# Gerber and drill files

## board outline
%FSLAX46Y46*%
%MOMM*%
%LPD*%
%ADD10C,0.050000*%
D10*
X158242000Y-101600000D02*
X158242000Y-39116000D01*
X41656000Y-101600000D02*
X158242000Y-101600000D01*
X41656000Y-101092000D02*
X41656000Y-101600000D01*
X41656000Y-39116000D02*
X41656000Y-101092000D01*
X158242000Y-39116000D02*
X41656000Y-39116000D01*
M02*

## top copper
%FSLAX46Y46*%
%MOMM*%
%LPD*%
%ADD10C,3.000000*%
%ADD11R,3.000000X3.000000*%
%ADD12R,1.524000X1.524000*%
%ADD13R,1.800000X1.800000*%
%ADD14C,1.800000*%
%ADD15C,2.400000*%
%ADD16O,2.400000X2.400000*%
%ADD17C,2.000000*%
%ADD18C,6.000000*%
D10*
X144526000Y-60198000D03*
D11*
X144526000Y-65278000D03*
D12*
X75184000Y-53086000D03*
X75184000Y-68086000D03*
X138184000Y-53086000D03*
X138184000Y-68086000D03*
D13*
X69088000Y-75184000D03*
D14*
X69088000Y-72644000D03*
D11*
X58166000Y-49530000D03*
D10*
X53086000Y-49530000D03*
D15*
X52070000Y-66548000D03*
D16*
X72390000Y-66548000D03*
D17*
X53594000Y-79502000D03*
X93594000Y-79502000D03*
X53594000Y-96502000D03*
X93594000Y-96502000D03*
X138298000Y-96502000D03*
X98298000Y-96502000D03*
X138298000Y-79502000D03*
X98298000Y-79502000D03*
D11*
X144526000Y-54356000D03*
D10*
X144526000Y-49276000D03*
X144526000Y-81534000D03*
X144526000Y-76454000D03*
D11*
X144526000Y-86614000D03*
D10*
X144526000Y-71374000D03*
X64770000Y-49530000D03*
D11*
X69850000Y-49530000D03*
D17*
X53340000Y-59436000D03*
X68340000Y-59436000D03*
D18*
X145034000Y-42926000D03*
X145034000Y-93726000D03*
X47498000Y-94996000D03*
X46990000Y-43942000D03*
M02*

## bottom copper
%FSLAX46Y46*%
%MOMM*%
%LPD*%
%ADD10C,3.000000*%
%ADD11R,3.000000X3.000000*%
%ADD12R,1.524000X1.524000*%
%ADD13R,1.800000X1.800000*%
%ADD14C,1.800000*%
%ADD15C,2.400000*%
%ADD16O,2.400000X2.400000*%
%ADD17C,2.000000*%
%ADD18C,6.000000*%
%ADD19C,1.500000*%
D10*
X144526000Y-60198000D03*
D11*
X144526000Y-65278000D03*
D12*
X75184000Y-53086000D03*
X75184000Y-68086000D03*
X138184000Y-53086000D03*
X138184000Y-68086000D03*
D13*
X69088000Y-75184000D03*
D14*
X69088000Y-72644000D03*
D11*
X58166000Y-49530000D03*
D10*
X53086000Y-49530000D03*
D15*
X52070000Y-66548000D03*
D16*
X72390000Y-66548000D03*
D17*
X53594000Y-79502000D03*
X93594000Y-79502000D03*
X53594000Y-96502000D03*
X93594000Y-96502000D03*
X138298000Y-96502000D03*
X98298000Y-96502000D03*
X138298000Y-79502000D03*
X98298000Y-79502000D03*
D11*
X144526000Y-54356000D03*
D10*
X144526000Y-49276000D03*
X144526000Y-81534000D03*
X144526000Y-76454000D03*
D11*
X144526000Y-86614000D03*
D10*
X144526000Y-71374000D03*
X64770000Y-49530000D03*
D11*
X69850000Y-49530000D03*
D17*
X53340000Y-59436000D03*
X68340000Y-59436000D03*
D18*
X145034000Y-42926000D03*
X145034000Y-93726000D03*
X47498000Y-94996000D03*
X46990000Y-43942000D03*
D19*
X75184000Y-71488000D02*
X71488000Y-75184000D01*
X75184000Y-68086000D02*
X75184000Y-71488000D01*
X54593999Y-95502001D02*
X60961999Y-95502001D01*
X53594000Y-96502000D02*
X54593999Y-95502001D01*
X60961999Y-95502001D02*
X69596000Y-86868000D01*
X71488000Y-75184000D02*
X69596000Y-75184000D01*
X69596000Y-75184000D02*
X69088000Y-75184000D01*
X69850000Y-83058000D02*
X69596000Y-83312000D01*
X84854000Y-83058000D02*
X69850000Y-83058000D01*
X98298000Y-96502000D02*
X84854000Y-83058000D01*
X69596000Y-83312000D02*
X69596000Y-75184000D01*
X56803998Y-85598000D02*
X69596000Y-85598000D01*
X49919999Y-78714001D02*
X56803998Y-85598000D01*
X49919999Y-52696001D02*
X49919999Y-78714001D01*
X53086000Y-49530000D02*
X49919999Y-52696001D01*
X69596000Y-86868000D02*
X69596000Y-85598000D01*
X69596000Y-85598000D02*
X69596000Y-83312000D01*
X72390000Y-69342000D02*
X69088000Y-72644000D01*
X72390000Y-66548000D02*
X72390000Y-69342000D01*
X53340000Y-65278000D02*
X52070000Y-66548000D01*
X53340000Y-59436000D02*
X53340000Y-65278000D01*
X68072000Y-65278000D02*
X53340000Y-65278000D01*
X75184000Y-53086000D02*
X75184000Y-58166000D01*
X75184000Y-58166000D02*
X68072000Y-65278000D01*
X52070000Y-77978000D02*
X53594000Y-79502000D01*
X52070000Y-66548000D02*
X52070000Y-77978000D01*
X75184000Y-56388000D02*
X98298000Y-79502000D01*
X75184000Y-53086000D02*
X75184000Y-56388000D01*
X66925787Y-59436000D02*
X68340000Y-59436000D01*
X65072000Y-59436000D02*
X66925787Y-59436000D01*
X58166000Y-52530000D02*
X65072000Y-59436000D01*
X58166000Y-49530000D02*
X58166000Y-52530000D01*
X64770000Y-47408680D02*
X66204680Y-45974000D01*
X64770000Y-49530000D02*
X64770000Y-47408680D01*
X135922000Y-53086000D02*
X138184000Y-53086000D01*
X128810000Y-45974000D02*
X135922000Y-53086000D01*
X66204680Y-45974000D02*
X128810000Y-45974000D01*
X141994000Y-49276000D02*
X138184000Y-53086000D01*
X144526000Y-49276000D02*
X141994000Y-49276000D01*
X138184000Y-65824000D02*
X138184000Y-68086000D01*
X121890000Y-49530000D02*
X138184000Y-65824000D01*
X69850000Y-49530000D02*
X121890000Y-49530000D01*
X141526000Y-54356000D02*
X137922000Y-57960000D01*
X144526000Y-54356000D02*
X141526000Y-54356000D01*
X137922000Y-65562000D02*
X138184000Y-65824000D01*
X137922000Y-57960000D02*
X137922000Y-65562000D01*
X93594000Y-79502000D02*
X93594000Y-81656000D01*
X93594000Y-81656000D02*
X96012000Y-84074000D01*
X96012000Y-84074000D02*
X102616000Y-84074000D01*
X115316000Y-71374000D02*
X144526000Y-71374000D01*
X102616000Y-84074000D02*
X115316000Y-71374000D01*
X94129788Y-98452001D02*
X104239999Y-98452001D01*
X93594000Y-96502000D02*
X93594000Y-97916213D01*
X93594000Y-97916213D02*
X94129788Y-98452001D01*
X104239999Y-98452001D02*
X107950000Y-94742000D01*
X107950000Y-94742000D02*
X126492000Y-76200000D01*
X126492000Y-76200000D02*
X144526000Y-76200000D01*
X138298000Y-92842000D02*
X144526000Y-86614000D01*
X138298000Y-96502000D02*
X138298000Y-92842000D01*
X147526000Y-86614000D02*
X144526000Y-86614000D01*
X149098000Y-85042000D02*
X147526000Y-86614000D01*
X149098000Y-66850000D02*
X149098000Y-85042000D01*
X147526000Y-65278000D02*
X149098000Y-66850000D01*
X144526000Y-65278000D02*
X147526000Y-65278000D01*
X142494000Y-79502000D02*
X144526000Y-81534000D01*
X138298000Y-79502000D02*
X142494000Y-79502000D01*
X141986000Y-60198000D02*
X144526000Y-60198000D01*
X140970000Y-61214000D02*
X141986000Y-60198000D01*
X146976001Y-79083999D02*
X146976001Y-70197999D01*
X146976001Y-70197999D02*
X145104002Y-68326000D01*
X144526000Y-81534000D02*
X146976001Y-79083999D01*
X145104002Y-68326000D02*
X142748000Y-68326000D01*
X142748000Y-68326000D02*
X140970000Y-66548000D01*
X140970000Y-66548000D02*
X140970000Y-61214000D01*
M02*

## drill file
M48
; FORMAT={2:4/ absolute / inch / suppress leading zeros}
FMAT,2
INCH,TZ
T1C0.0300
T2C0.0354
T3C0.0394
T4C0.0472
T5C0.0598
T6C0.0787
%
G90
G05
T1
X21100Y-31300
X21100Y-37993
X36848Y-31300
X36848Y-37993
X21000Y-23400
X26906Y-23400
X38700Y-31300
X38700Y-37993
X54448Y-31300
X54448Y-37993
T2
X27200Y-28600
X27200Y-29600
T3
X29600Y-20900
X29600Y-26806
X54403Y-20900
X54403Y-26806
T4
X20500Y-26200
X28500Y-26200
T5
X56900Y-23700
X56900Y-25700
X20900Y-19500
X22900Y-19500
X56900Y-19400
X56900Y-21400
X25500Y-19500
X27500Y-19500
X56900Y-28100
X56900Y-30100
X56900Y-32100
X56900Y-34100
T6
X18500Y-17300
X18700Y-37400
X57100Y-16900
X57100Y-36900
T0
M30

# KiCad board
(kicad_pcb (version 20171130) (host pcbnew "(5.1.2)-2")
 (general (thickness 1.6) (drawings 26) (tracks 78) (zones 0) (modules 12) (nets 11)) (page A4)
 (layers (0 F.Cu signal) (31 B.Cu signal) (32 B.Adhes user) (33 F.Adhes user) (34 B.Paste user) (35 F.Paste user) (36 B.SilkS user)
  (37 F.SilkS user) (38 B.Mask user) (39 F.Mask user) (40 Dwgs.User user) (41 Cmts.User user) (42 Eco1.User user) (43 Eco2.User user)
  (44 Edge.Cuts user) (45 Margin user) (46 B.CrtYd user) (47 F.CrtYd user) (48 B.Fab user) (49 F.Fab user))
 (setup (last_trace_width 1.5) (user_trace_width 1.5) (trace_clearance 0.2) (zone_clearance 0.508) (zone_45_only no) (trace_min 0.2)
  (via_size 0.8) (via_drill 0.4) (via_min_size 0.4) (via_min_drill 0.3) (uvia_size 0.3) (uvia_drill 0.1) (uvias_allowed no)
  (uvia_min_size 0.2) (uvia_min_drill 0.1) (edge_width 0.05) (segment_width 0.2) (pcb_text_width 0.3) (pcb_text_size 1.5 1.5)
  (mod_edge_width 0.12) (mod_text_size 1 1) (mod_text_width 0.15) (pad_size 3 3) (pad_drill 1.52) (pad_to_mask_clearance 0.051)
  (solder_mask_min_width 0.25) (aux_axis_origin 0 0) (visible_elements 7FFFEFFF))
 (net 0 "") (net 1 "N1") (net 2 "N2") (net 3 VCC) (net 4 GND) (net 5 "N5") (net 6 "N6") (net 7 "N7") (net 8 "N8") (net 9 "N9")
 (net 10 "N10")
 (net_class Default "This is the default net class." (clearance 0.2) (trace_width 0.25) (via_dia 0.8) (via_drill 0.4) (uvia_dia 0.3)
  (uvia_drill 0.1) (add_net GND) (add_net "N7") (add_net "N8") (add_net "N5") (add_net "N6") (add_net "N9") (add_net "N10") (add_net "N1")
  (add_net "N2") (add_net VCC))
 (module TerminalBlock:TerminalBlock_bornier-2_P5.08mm (layer F.Cu) (at 144.526 65.278 90)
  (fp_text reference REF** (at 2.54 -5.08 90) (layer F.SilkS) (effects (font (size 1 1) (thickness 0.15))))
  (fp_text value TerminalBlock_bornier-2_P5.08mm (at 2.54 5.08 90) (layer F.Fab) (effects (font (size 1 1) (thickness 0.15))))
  (pad 2 thru_hole circle (at 5.08 0 90) (size 3 3) (drill 1.52) (layers *.Cu *.Mask) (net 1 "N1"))
  (pad 1 thru_hole rect (at 0 0 90) (size 3 3) (drill 1.52) (layers *.Cu *.Mask) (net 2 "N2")))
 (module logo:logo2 (layer F.Cu) (at 105.918 60.198)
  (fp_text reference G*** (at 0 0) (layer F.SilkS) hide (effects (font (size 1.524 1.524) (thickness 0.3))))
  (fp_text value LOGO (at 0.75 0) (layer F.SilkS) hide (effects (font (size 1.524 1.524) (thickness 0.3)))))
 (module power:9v (layer F.Cu) (at 75.184 53.086)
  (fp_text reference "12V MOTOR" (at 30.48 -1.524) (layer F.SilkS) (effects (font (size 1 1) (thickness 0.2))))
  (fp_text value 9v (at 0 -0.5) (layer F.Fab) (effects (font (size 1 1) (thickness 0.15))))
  (pad 1 thru_hole rect (at 0 0) (size 1.524 1.524) (drill 1) (layers *.Cu *.Mask) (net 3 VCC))
  (pad 3 thru_hole rect (at 0 15) (size 1.524 1.524) (drill 1) (layers *.Cu *.Mask) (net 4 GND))
  (pad 2 thru_hole rect (at 63 0) (size 1.524 1.524) (drill 1) (layers *.Cu *.Mask) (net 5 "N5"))
  (pad 4 thru_hole rect (at 63 15) (size 1.524 1.524) (drill 1) (layers *.Cu *.Mask) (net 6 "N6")))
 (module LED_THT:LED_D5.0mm (layer F.Cu) (at 69.088 75.184 90)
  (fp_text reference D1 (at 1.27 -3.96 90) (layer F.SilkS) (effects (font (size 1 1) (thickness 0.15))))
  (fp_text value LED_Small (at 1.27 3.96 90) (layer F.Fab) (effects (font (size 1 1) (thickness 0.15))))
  (pad 1 thru_hole rect (at 0 0 90) (size 1.8 1.8) (drill 0.9) (layers *.Cu *.Mask) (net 4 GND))
  (pad 2 thru_hole circle (at 2.54 0 90) (size 1.8 1.8) (drill 0.9) (layers *.Cu *.Mask) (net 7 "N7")))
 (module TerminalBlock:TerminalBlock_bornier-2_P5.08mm (layer F.Cu) (at 58.166 49.53 180)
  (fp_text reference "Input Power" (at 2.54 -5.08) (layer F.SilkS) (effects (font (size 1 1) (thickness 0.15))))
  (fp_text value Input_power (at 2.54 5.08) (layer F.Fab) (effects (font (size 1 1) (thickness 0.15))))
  (pad 1 thru_hole rect (at 0 0 180) (size 3 3) (drill 1.52) (layers *.Cu *.Mask) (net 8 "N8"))
  (pad 2 thru_hole circle (at 5.08 0 180) (size 3 3) (drill 1.52) (layers *.Cu *.Mask) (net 4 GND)))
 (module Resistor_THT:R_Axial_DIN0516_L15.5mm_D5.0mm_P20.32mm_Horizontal (layer F.Cu) (at 52.07 66.548)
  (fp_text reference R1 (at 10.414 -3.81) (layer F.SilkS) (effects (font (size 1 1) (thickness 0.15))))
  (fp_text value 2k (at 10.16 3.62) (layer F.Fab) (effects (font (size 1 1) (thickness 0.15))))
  (pad 1 thru_hole circle (at 0 0) (size 2.4 2.4) (drill 1.2) (layers *.Cu *.Mask) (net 3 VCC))
  (pad 2 thru_hole oval (at 20.32 0) (size 2.4 2.4) (drill 1.2) (layers *.Cu *.Mask) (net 7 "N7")))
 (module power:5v (layer F.Cu) (at 53.594 79.502)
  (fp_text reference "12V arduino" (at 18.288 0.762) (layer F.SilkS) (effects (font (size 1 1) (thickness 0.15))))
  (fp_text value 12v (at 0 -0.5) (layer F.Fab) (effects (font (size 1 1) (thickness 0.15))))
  (pad 1 thru_hole circle (at 0 0) (size 2 2) (drill 0.762) (layers *.Cu *.Mask) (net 3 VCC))
  (pad 2 thru_hole circle (at 40 0) (size 2 2) (drill 0.762) (layers *.Cu *.Mask) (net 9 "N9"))
  (pad 3 thru_hole circle (at 0 17) (size 2 2) (drill 0.762) (layers *.Cu *.Mask) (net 4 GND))
  (pad 4 thru_hole circle (at 40 17) (size 2 2) (drill 0.762) (layers *.Cu *.Mask) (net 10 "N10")))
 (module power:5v (layer F.Cu) (at 98.298 79.502)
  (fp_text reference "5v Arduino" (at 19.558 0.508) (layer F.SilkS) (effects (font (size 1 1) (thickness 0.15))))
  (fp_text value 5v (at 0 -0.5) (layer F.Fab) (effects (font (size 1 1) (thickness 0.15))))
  (pad 4 thru_hole circle (at 40 17) (size 2 2) (drill 0.762) (layers *.Cu *.Mask) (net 2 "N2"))
  (pad 3 thru_hole circle (at 0 17) (size 2 2) (drill 0.762) (layers *.Cu *.Mask) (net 4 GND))
  (pad 2 thru_hole circle (at 40 0) (size 2 2) (drill 0.762) (layers *.Cu *.Mask) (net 1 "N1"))
  (pad 1 thru_hole circle (at 0 0) (size 2 2) (drill 0.762) (layers *.Cu *.Mask) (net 3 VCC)))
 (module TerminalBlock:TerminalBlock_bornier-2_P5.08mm (layer F.Cu) (at 144.526 54.356 90)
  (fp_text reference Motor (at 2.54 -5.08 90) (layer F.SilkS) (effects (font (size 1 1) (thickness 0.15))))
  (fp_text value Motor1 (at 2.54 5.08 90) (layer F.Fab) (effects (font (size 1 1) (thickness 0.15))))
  (pad 1 thru_hole rect (at 0 0 90) (size 3 3) (drill 1.52) (layers *.Cu *.Mask) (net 6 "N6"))
  (pad 2 thru_hole circle (at 5.08 0 90) (size 3 3) (drill 1.52) (layers *.Cu *.Mask) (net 5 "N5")))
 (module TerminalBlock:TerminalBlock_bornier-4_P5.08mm (layer F.Cu) (at 144.526 86.614 90)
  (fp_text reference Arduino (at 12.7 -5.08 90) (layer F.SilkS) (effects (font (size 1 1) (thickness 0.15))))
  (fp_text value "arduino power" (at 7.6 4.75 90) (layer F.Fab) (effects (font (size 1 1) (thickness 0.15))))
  (pad 2 thru_hole circle (at 5.08 0 90) (size 3 3) (drill 1.52) (layers *.Cu *.Mask) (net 1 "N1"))
  (pad 3 thru_hole circle (at 10.16 0 90) (size 3 3) (drill 1.52) (layers *.Cu *.Mask) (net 10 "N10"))
  (pad 1 thru_hole rect (at 0 0 90) (size 3 3) (drill 1.52) (layers *.Cu *.Mask) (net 2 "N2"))
  (pad 4 thru_hole circle (at 15.24 0 90) (size 3 3) (drill 1.52) (layers *.Cu *.Mask) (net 9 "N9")))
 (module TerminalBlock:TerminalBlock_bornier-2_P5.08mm (layer F.Cu) (at 69.85 49.53 180)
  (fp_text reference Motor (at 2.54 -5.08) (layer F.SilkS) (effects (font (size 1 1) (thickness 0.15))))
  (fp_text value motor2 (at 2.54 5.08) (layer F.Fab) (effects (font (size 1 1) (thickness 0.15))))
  (pad 2 thru_hole circle (at 5.08 0 180) (size 3 3) (drill 1.52) (layers *.Cu *.Mask) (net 5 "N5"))
  (pad 1 thru_hole rect (at 0 0 180) (size 3 3) (drill 1.52) (layers *.Cu *.Mask) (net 6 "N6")))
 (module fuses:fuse (layer F.Cu) (at 53.34 59.436)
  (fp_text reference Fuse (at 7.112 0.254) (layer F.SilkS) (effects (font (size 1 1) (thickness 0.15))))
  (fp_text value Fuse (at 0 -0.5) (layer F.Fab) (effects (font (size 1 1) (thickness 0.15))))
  (pad 1 thru_hole circle (at 0 0) (size 2 2) (drill 0.762) (layers *.Cu *.Mask) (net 3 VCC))
  (pad 2 thru_hole circle (at 15 0) (size 2 2) (drill 0.762) (layers *.Cu *.Mask) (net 8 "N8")))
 (gr_line (start 158.242 101.6) (end 158.242 39.116) (layer Edge.Cuts) (width 0.05))
 (gr_line (start 41.656 101.6) (end 158.242 101.6) (layer Edge.Cuts) (width 0.05))
 (gr_line (start 41.656 101.092) (end 41.656 101.6) (layer Edge.Cuts) (width 0.05))
 (gr_line (start 41.656 39.116) (end 41.656 101.092) (layer Edge.Cuts) (width 0.05))
 (gr_line (start 158.242 39.116) (end 41.656 39.116) (layer Edge.Cuts) (width 0.05))
 (via (at 145.034 42.926) (size 6) (drill 2) (layers F.Cu B.Cu) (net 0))
 (via (at 145.034 93.726) (size 6) (drill 2) (layers F.Cu B.Cu) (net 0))
 (via (at 47.498 94.996) (size 6) (drill 2) (layers F.Cu B.Cu) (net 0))
 (via (at 46.99 43.942) (size 6) (drill 2) (layers F.Cu B.Cu) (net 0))
 (segment (start 75.184 71.488) (end 71.488 75.184) (width 1.5) (layer B.Cu) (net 4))
 (segment (start 75.184 68.086) (end 75.184 71.488) (width 1.5) (layer B.Cu) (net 4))
 (segment (start 54.593999 95.502001) (end 60.961999 95.502001) (width 1.5) (layer B.Cu) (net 4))
 (segment (start 53.594 96.502) (end 54.593999 95.502001) (width 1.5) (layer B.Cu) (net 4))
 (segment (start 60.961999 95.502001) (end 69.596 86.868) (width 1.5) (layer B.Cu) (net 4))
 (segment (start 71.488 75.184) (end 69.596 75.184) (width 1.5) (layer B.Cu) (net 4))
 (segment (start 69.596 75.184) (end 69.088 75.184) (width 1.5) (layer B.Cu) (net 4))
 (segment (start 69.85 83.058) (end 69.596 83.312) (width 1.5) (layer B.Cu) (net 4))
 (segment (start 84.854 83.058) (end 69.85 83.058) (width 1.5) (layer B.Cu) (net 4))
 (segment (start 98.298 96.502) (end 84.854 83.058) (width 1.5) (layer B.Cu) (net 4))
 (segment (start 69.596 83.312) (end 69.596 75.184) (width 1.5) (layer B.Cu) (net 4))
 (segment (start 56.803998 85.598) (end 69.596 85.598) (width 1.5) (layer B.Cu) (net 4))
 (segment (start 49.919999 78.714001) (end 56.803998 85.598) (width 1.5) (layer B.Cu) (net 4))
 (segment (start 49.919999 52.696001) (end 49.919999 78.714001) (width 1.5) (layer B.Cu) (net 4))
 (segment (start 53.086 49.53) (end 49.919999 52.696001) (width 1.5) (layer B.Cu) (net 4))
 (segment (start 69.596 86.868) (end 69.596 85.598) (width 1.5) (layer B.Cu) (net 4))
 (segment (start 69.596 85.598) (end 69.596 83.312) (width 1.5) (layer B.Cu) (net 4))
 (segment (start 72.39 69.342) (end 69.088 72.644) (width 1.5) (layer B.Cu) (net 7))
 (segment (start 72.39 66.548) (end 72.39 69.342) (width 1.5) (layer B.Cu) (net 7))
 (segment (start 53.34 65.278) (end 52.07 66.548) (width 1.5) (layer B.Cu) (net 3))
 (segment (start 53.34 59.436) (end 53.34 65.278) (width 1.5) (layer B.Cu) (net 3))
 (segment (start 68.072 65.278) (end 53.34 65.278) (width 1.5) (layer B.Cu) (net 3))
 (segment (start 75.184 53.086) (end 75.184 58.166) (width 1.5) (layer B.Cu) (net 3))
 (segment (start 75.184 58.166) (end 68.072 65.278) (width 1.5) (layer B.Cu) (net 3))
 (segment (start 52.07 77.978) (end 53.594 79.502) (width 1.5) (layer B.Cu) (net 3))
 (segment (start 52.07 66.548) (end 52.07 77.978) (width 1.5) (layer B.Cu) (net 3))
 (segment (start 75.184 56.388) (end 98.298 79.502) (width 1.5) (layer B.Cu) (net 3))
 (segment (start 75.184 53.086) (end 75.184 56.388) (width 1.5) (layer B.Cu) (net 3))
 (segment (start 66.925787 59.436) (end 68.34 59.436) (width 1.5) (layer B.Cu) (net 8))
 (segment (start 65.072 59.436) (end 66.925787 59.436) (width 1.5) (layer B.Cu) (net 8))
 (segment (start 58.166 52.53) (end 65.072 59.436) (width 1.5) (layer B.Cu) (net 8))
 (segment (start 58.166 49.53) (end 58.166 52.53) (width 1.5) (layer B.Cu) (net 8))
 (segment (start 64.77 47.40868) (end 66.20468 45.974) (width 1.5) (layer B.Cu) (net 5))
 (segment (start 64.77 49.53) (end 64.77 47.40868) (width 1.5) (layer B.Cu) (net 5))
 (segment (start 135.922 53.086) (end 138.184 53.086) (width 1.5) (layer B.Cu) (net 5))
 (segment (start 128.81 45.974) (end 135.922 53.086) (width 1.5) (layer B.Cu) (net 5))
 (segment (start 66.20468 45.974) (end 128.81 45.974) (width 1.5) (layer B.Cu) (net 5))
 (segment (start 141.994 49.276) (end 138.184 53.086) (width 1.5) (layer B.Cu) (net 5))
 (segment (start 144.526 49.276) (end 141.994 49.276) (width 1.5) (layer B.Cu) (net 5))
 (segment (start 138.184 65.824) (end 138.184 68.086) (width 1.5) (layer B.Cu) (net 6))
 (segment (start 121.89 49.53) (end 138.184 65.824) (width 1.5) (layer B.Cu) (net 6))
 (segment (start 69.85 49.53) (end 121.89 49.53) (width 1.5) (layer B.Cu) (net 6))
 (segment (start 141.526 54.356) (end 137.922 57.96) (width 1.5) (layer B.Cu) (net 6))
 (segment (start 144.526 54.356) (end 141.526 54.356) (width 1.5) (layer B.Cu) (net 6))
 (segment (start 137.922 65.562) (end 138.184 65.824) (width 1.5) (layer B.Cu) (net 6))
 (segment (start 137.922 57.96) (end 137.922 65.562) (width 1.5) (layer B.Cu) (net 6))
 (segment (start 93.594 79.502) (end 93.594 81.656) (width 1.5) (layer B.Cu) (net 9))
 (segment (start 93.594 81.656) (end 96.012 84.074) (width 1.5) (layer B.Cu) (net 9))
 (segment (start 96.012 84.074) (end 102.616 84.074) (width 1.5) (layer B.Cu) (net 9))
 (segment (start 115.316 71.374) (end 144.526 71.374) (width 1.5) (layer B.Cu) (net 9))
 (segment (start 102.616 84.074) (end 115.316 71.374) (width 1.5) (layer B.Cu) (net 9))
 (segment (start 94.129788 98.452001) (end 104.239999 98.452001) (width 1.5) (layer B.Cu) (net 10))
 (segment (start 93.594 96.502) (end 93.594 97.916213) (width 1.5) (layer B.Cu) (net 10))
 (segment (start 93.594 97.916213) (end 94.129788 98.452001) (width 1.5) (layer B.Cu) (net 10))
 (segment (start 104.239999 98.452001) (end 107.95 94.742) (width 1.5) (layer B.Cu) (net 10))
 (segment (start 107.95 94.742) (end 126.492 76.2) (width 1.5) (layer B.Cu) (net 10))
 (segment (start 126.492 76.2) (end 144.526 76.2) (width 1.5) (layer B.Cu) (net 10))
 (segment (start 138.298 92.842) (end 144.526 86.614) (width 1.5) (layer B.Cu) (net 2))
 (segment (start 138.298 96.502) (end 138.298 92.842) (width 1.5) (layer B.Cu) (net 2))
 (segment (start 147.526 86.614) (end 144.526 86.614) (width 1.5) (layer B.Cu) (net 2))
 (segment (start 149.098 85.042) (end 147.526 86.614) (width 1.5) (layer B.Cu) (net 2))
 (segment (start 149.098 66.85) (end 149.098 85.042) (width 1.5) (layer B.Cu) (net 2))
 (segment (start 147.526 65.278) (end 149.098 66.85) (width 1.5) (layer B.Cu) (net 2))
 (segment (start 144.526 65.278) (end 147.526 65.278) (width 1.5) (layer B.Cu) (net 2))
 (segment (start 142.494 79.502) (end 144.526 81.534) (width 1.5) (layer B.Cu) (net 1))
 (segment (start 138.298 79.502) (end 142.494 79.502) (width 1.5) (layer B.Cu) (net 1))
 (segment (start 141.986 60.198) (end 144.526 60.198) (width 1.5) (layer B.Cu) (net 1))
 (segment (start 140.97 61.214) (end 141.986 60.198) (width 1.5) (layer B.Cu) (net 1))
 (segment (start 146.976001 79.083999) (end 146.976001 70.197999) (width 1.5) (layer B.Cu) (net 1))
 (segment (start 146.976001 70.197999) (end 145.104002 68.326) (width 1.5) (layer B.Cu) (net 1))
 (segment (start 144.526 81.534) (end 146.976001 79.083999) (width 1.5) (layer B.Cu) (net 1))
 (segment (start 145.104002 68.326) (end 142.748 68.326) (width 1.5) (layer B.Cu) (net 1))
 (segment (start 142.748 68.326) (end 140.97 66.548) (width 1.5) (layer B.Cu) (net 1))
 (segment (start 140.97 66.548) (end 140.97 61.214) (width 1.5) (layer B.Cu) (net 1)))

